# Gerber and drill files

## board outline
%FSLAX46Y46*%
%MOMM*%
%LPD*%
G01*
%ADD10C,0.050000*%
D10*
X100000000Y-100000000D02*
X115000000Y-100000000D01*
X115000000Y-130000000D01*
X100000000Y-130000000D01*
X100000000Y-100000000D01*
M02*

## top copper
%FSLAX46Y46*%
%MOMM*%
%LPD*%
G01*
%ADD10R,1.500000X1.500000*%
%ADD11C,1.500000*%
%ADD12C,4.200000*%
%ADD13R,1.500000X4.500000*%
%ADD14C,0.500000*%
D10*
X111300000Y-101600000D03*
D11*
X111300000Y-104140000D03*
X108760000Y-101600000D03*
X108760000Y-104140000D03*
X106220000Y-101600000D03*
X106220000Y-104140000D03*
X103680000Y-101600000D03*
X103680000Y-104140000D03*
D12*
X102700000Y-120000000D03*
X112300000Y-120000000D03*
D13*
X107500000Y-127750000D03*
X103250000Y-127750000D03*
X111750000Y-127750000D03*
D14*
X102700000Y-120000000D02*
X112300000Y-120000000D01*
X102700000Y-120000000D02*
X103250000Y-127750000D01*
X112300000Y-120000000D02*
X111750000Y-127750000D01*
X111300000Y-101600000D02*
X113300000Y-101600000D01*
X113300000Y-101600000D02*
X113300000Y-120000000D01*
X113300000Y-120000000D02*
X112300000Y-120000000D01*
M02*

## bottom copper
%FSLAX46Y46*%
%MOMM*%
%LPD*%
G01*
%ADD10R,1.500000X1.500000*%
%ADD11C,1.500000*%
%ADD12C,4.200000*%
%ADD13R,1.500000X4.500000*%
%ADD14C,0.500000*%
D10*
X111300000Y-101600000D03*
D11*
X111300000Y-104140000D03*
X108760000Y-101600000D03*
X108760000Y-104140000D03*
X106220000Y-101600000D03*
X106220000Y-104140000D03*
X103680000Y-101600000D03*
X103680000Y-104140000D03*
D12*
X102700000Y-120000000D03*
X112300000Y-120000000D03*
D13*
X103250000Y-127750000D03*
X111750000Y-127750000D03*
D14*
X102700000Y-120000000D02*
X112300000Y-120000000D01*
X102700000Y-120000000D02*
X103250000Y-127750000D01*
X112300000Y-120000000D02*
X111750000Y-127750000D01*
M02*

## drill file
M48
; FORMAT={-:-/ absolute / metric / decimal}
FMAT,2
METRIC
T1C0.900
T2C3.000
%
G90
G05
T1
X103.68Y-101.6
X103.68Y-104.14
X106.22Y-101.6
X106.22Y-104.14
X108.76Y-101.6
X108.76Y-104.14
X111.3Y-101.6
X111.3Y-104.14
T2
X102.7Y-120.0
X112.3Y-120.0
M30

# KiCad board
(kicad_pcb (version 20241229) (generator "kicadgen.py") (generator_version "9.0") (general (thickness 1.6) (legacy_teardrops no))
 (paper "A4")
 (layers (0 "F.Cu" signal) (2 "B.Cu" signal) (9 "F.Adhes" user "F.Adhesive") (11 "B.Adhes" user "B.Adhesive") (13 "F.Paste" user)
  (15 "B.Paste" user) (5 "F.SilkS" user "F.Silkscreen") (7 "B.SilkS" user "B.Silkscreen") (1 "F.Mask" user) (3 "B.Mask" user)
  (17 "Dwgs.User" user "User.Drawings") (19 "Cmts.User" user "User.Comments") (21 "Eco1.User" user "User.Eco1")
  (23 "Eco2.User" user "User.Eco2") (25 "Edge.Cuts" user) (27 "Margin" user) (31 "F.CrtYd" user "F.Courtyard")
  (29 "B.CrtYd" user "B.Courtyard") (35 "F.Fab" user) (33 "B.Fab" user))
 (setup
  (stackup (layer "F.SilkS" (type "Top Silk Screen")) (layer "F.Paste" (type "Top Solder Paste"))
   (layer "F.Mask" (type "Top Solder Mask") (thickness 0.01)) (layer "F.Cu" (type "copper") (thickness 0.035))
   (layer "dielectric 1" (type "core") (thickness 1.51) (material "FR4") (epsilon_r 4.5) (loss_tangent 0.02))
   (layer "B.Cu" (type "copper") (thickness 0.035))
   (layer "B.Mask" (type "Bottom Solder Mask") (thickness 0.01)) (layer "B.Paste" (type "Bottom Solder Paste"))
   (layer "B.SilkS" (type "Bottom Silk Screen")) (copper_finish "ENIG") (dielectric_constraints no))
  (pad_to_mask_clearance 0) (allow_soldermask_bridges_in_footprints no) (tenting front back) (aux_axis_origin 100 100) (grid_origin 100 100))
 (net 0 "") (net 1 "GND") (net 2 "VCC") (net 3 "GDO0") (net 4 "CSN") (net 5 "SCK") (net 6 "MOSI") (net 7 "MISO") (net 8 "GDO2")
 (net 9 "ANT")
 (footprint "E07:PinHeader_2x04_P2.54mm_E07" (layer "F.Cu") (at 111.3 101.6)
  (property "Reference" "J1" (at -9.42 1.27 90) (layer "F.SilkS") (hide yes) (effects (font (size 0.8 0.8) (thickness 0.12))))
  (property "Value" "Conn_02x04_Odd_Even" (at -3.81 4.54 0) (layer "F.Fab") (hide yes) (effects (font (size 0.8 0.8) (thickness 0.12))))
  (pad "1" thru_hole rect (at 0 0) (size 1.5 1.5) (drill 0.9) (layers "*.Cu" "*.Mask") (remove_unused_layers no) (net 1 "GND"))
  (pad "2" thru_hole circle (at 0 2.54) (size 1.5 1.5) (drill 0.9) (layers "*.Cu" "*.Mask") (remove_unused_layers no) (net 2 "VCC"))
  (pad "3" thru_hole circle (at -2.54 0) (size 1.5 1.5) (drill 0.9) (layers "*.Cu" "*.Mask") (remove_unused_layers no) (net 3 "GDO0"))
  (pad "4" thru_hole circle (at -2.54 2.54) (size 1.5 1.5) (drill 0.9) (layers "*.Cu" "*.Mask") (remove_unused_layers no) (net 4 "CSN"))
  (pad "5" thru_hole circle (at -5.08 0) (size 1.5 1.5) (drill 0.9) (layers "*.Cu" "*.Mask") (remove_unused_layers no) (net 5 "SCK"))
  (pad "6" thru_hole circle (at -5.08 2.54) (size 1.5 1.5) (drill 0.9) (layers "*.Cu" "*.Mask") (remove_unused_layers no) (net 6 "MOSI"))
  (pad "7" thru_hole circle (at -7.62 0) (size 1.5 1.5) (drill 0.9) (layers "*.Cu" "*.Mask") (remove_unused_layers no) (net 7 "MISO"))
  (pad "8" thru_hole circle (at -7.62 2.54) (size 1.5 1.5) (drill 0.9) (layers "*.Cu" "*.Mask") (remove_unused_layers no) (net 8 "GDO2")))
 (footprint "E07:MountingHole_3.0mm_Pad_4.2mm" (layer "F.Cu") (at 102.7 120)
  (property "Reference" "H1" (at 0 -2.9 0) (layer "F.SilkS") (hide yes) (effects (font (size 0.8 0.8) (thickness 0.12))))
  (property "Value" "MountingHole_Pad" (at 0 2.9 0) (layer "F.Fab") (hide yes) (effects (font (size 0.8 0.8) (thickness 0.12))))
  (pad "1" thru_hole circle (at 0 0) (size 4.2 4.2) (drill 3) (layers "*.Cu" "*.Mask") (remove_unused_layers no) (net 1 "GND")))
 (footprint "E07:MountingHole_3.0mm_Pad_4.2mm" (layer "F.Cu") (at 112.3 120)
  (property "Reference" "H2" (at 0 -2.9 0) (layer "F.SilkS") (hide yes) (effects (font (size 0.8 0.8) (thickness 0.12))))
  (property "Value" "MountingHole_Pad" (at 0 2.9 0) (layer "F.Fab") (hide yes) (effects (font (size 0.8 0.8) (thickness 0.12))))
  (pad "1" thru_hole circle (at 0 0) (size 4.2 4.2) (drill 3) (layers "*.Cu" "*.Mask") (remove_unused_layers no) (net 1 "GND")))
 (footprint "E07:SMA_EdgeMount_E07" (layer "F.Cu") (at 107.5 130)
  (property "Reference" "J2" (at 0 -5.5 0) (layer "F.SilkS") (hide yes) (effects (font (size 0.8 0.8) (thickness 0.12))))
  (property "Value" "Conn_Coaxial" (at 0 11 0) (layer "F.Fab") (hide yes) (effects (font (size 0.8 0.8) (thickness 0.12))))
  (pad "1" smd rect (at 0 -2.25) (size 1.5 4.5) (layers "F.Cu" "F.Mask" "F.Paste") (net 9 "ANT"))
  (pad "2" smd rect (at -4.25 -2.25) (size 1.5 4.5) (layers "F.Cu" "F.Mask" "F.Paste") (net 1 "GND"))
  (pad "2" smd rect (at -4.25 -2.25) (size 1.5 4.5) (layers "B.Cu" "B.Mask" "B.Paste") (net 1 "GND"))
  (pad "2" smd rect (at 4.25 -2.25) (size 1.5 4.5) (layers "F.Cu" "F.Mask" "F.Paste") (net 1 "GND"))
  (pad "2" smd rect (at 4.25 -2.25) (size 1.5 4.5) (layers "B.Cu" "B.Mask" "B.Paste") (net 1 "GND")))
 (gr_rect (start 100 100) (end 115 130) (stroke (width 0.05) (type solid)) (fill no) (layer "Edge.Cuts"))
 (segment (start 102.7 120) (end 112.3 120) (width 0.5) (layer "F.Cu") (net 1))
 (segment (start 102.7 120) (end 103.25 127.75) (width 0.5) (layer "F.Cu") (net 1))
 (segment (start 112.3 120) (end 111.75 127.75) (width 0.5) (layer "F.Cu") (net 1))
 (segment (start 102.7 120) (end 112.3 120) (width 0.5) (layer "B.Cu") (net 1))
 (segment (start 102.7 120) (end 103.25 127.75) (width 0.5) (layer "B.Cu") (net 1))
 (segment (start 112.3 120) (end 111.75 127.75) (width 0.5) (layer "B.Cu") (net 1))
 (segment (start 111.3 101.6) (end 113.3 101.6) (width 0.5) (layer "F.Cu") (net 1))
 (segment (start 113.3 101.6) (end 113.3 120) (width 0.5) (layer "F.Cu") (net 1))
 (segment (start 113.3 120) (end 112.3 120) (width 0.5) (layer "F.Cu") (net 1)))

